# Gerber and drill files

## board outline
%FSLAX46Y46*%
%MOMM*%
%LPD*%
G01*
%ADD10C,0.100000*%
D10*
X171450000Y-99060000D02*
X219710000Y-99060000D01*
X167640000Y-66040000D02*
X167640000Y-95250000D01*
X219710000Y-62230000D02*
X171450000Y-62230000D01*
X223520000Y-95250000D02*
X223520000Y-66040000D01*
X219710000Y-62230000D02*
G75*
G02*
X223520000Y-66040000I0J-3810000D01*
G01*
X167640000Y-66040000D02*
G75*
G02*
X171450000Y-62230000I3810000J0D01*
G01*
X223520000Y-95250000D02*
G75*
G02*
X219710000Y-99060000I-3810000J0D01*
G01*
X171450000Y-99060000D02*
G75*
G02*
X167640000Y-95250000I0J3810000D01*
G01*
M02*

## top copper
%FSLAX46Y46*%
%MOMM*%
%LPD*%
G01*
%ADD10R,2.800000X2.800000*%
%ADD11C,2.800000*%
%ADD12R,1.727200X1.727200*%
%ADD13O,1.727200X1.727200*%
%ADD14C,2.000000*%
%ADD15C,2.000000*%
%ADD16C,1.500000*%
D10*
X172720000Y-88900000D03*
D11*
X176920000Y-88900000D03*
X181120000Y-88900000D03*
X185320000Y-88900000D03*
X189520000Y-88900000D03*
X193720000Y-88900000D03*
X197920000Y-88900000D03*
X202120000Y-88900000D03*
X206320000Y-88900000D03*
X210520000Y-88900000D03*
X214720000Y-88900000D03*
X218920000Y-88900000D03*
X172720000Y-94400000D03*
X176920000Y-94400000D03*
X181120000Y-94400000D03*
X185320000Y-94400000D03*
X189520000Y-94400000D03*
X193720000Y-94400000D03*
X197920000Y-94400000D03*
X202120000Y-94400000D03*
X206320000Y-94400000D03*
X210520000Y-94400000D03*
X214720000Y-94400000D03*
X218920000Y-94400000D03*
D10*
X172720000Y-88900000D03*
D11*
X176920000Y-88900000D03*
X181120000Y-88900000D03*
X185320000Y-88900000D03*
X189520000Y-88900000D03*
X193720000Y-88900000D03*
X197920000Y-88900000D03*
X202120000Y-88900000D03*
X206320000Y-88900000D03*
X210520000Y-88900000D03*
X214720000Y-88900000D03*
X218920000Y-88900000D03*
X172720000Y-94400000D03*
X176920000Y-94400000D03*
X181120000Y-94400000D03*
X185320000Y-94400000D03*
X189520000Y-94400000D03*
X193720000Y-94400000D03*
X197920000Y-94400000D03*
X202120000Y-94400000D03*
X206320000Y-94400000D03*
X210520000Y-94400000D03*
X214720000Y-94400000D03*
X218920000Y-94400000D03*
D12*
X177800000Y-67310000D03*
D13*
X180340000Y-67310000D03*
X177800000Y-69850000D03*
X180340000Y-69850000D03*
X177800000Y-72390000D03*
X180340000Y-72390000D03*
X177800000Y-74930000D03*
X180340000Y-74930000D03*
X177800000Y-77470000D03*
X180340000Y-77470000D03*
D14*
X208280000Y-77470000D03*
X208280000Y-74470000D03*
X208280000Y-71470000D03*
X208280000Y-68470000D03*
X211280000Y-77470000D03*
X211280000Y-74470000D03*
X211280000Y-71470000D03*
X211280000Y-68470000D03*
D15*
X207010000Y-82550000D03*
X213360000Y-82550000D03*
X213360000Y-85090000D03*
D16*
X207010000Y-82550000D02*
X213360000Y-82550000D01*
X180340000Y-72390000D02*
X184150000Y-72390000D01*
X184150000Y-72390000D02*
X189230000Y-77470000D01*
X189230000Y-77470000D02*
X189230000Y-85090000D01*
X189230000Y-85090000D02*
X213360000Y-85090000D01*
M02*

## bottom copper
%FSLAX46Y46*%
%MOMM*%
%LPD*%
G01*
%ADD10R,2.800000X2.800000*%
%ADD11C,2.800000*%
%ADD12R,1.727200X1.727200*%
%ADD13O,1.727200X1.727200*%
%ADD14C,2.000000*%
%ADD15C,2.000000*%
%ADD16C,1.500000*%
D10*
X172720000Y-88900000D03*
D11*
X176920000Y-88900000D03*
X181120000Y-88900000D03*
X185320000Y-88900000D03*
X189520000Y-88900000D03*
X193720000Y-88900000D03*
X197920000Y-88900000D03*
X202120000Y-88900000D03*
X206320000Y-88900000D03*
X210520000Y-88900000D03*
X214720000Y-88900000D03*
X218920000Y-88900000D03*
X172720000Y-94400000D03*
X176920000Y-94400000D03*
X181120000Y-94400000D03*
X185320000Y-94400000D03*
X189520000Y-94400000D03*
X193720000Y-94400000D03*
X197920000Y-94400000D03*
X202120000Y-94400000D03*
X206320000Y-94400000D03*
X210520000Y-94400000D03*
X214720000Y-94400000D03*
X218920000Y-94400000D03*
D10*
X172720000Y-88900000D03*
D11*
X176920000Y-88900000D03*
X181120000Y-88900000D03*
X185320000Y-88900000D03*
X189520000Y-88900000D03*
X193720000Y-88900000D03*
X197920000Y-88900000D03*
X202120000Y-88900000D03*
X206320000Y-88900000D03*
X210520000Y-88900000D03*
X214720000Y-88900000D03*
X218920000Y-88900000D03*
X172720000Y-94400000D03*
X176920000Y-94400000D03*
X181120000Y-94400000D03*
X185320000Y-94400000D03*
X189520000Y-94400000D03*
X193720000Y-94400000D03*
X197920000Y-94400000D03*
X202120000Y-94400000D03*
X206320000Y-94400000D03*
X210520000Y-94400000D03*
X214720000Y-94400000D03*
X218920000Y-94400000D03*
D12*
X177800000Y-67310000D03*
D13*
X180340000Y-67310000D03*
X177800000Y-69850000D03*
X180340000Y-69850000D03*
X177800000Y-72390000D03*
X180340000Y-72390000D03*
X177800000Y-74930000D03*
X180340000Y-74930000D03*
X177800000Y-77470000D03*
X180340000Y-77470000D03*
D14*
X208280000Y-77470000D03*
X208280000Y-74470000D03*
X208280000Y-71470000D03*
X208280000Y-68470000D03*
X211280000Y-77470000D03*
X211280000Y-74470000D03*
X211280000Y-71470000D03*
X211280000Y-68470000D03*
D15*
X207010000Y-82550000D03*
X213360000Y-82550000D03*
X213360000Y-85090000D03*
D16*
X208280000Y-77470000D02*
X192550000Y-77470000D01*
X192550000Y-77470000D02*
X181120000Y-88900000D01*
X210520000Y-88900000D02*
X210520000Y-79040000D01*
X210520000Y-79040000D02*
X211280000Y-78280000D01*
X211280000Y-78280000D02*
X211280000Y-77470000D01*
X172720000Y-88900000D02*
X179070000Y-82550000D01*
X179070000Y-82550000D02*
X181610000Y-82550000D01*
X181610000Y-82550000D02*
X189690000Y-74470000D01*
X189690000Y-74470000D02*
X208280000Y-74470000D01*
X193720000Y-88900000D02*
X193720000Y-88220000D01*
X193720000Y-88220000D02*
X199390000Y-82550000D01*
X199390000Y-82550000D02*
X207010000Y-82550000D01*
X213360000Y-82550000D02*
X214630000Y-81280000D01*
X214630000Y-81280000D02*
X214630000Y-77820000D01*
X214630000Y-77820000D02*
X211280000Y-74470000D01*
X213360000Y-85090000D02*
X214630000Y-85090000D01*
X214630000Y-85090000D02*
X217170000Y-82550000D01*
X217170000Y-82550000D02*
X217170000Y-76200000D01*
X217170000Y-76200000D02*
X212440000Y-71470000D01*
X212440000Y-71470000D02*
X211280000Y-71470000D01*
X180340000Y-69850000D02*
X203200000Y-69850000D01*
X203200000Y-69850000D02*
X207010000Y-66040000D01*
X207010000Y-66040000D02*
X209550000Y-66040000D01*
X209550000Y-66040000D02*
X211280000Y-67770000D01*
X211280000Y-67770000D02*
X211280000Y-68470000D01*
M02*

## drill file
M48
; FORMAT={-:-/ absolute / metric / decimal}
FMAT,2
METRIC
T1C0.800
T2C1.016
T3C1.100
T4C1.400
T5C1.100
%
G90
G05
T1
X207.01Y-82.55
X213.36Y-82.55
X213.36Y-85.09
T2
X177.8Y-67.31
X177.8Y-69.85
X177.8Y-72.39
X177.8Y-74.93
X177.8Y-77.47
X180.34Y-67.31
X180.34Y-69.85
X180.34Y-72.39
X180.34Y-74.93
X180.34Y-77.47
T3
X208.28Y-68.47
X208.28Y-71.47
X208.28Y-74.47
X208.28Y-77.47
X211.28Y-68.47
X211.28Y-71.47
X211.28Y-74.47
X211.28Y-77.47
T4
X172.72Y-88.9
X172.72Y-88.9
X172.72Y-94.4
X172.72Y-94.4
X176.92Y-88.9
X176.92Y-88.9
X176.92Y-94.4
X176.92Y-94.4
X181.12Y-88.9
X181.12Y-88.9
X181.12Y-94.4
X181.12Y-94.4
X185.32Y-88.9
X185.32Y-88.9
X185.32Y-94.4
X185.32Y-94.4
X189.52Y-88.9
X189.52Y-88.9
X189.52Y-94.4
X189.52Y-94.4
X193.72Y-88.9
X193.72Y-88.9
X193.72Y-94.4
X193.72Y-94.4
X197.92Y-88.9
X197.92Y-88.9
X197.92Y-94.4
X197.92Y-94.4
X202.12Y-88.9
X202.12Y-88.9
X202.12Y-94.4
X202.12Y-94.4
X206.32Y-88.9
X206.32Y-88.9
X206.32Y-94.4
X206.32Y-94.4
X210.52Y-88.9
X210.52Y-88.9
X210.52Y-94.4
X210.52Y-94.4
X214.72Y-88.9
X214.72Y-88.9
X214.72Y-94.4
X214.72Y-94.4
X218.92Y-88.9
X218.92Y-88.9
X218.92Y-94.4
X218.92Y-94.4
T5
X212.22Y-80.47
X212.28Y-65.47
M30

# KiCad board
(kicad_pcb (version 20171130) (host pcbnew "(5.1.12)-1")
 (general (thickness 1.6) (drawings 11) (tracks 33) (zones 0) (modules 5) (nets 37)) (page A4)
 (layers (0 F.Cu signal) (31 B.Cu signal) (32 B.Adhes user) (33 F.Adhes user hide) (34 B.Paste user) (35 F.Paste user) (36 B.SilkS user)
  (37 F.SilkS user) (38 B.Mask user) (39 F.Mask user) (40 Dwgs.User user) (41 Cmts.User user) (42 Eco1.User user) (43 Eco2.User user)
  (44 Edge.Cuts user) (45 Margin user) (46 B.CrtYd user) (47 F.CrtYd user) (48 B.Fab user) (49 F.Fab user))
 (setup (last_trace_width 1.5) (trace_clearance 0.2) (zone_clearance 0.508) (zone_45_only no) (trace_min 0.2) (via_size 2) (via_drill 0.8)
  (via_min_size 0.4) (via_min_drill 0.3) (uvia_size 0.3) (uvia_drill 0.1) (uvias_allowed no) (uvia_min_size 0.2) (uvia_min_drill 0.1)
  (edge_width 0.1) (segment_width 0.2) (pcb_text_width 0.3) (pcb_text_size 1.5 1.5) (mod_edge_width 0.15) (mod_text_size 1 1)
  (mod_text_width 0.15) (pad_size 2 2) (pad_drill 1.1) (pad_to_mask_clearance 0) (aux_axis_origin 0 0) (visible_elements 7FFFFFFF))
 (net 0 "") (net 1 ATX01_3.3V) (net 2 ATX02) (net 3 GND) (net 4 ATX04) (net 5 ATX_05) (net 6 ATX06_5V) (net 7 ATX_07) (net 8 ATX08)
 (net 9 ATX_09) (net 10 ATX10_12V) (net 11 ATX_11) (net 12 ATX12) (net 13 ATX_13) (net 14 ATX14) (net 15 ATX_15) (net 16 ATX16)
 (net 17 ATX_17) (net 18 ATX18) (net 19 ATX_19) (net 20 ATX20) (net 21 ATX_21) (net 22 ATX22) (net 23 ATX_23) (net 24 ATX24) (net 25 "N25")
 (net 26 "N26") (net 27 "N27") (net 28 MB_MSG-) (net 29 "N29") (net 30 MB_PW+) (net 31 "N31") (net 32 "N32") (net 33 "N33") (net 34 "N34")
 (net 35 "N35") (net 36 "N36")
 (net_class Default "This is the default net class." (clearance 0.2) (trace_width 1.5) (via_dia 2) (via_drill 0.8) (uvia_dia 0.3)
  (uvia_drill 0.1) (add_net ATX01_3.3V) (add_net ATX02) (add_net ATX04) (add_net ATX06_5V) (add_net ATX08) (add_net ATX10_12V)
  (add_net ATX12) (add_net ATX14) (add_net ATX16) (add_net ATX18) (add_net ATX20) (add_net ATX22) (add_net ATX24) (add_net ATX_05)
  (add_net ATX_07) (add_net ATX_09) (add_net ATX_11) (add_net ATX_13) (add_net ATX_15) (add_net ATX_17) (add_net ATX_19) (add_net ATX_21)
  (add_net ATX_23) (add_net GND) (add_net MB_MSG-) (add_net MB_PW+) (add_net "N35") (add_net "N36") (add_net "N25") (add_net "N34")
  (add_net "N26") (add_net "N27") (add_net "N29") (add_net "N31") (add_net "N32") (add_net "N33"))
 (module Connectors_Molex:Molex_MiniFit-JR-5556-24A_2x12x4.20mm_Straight (layer F.Cu) (at 172.72 88.9)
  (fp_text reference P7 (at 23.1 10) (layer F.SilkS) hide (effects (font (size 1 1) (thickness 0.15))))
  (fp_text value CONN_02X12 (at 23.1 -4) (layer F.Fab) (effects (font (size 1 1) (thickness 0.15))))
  (pad 1 thru_hole rect (at 0 0) (size 2.8 2.8) (drill 1.4) (layers *.Cu *.Mask) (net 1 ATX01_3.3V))
  (pad 2 thru_hole circle (at 4.2 0) (size 2.8 2.8) (drill 1.4) (layers *.Cu *.Mask) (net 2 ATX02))
  (pad 3 thru_hole circle (at 8.4 0) (size 2.8 2.8) (drill 1.4) (layers *.Cu *.Mask) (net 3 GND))
  (pad 4 thru_hole circle (at 12.6 0) (size 2.8 2.8) (drill 1.4) (layers *.Cu *.Mask) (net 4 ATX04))
  (pad 5 thru_hole circle (at 16.8 0) (size 2.8 2.8) (drill 1.4) (layers *.Cu *.Mask) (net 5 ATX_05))
  (pad 6 thru_hole circle (at 21 0) (size 2.8 2.8) (drill 1.4) (layers *.Cu *.Mask) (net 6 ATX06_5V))
  (pad 7 thru_hole circle (at 25.2 0) (size 2.8 2.8) (drill 1.4) (layers *.Cu *.Mask) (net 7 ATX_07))
  (pad 8 thru_hole circle (at 29.4 0) (size 2.8 2.8) (drill 1.4) (layers *.Cu *.Mask) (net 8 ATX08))
  (pad 9 thru_hole circle (at 33.6 0) (size 2.8 2.8) (drill 1.4) (layers *.Cu *.Mask) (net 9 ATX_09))
  (pad 10 thru_hole circle (at 37.8 0) (size 2.8 2.8) (drill 1.4) (layers *.Cu *.Mask) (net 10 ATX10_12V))
  (pad 11 thru_hole circle (at 42 0) (size 2.8 2.8) (drill 1.4) (layers *.Cu *.Mask) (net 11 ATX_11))
  (pad 12 thru_hole circle (at 46.2 0) (size 2.8 2.8) (drill 1.4) (layers *.Cu *.Mask) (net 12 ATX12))
  (pad 13 thru_hole circle (at 0 5.5) (size 2.8 2.8) (drill 1.4) (layers *.Cu *.Mask) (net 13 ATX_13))
  (pad 14 thru_hole circle (at 4.2 5.5) (size 2.8 2.8) (drill 1.4) (layers *.Cu *.Mask) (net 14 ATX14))
  (pad 15 thru_hole circle (at 8.4 5.5) (size 2.8 2.8) (drill 1.4) (layers *.Cu *.Mask) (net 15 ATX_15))
  (pad 16 thru_hole circle (at 12.6 5.5) (size 2.8 2.8) (drill 1.4) (layers *.Cu *.Mask) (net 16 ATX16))
  (pad 17 thru_hole circle (at 16.8 5.5) (size 2.8 2.8) (drill 1.4) (layers *.Cu *.Mask) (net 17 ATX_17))
  (pad 18 thru_hole circle (at 21 5.5) (size 2.8 2.8) (drill 1.4) (layers *.Cu *.Mask) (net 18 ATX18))
  (pad 19 thru_hole circle (at 25.2 5.5) (size 2.8 2.8) (drill 1.4) (layers *.Cu *.Mask) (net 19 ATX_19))
  (pad 20 thru_hole circle (at 29.4 5.5) (size 2.8 2.8) (drill 1.4) (layers *.Cu *.Mask) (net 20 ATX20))
  (pad 21 thru_hole circle (at 33.6 5.5) (size 2.8 2.8) (drill 1.4) (layers *.Cu *.Mask) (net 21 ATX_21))
  (pad 22 thru_hole circle (at 37.8 5.5) (size 2.8 2.8) (drill 1.4) (layers *.Cu *.Mask) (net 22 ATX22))
  (pad 23 thru_hole circle (at 42 5.5) (size 2.8 2.8) (drill 1.4) (layers *.Cu *.Mask) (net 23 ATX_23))
  (pad 24 thru_hole circle (at 46.2 5.5) (size 2.8 2.8) (drill 1.4) (layers *.Cu *.Mask) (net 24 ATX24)))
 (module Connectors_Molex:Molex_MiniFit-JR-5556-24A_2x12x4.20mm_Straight (layer F.Cu) (at 172.72 88.9)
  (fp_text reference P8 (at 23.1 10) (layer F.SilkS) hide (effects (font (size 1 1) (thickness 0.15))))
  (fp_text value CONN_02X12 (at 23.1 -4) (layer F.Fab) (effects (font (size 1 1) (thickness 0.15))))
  (pad 1 thru_hole rect (at 0 0) (size 2.8 2.8) (drill 1.4) (layers *.Cu *.Mask) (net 1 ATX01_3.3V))
  (pad 2 thru_hole circle (at 4.2 0) (size 2.8 2.8) (drill 1.4) (layers *.Cu *.Mask) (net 2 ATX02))
  (pad 3 thru_hole circle (at 8.4 0) (size 2.8 2.8) (drill 1.4) (layers *.Cu *.Mask) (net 3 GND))
  (pad 4 thru_hole circle (at 12.6 0) (size 2.8 2.8) (drill 1.4) (layers *.Cu *.Mask) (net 4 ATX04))
  (pad 5 thru_hole circle (at 16.8 0) (size 2.8 2.8) (drill 1.4) (layers *.Cu *.Mask) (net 5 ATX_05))
  (pad 6 thru_hole circle (at 21 0) (size 2.8 2.8) (drill 1.4) (layers *.Cu *.Mask) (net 6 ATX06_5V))
  (pad 7 thru_hole circle (at 25.2 0) (size 2.8 2.8) (drill 1.4) (layers *.Cu *.Mask) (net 7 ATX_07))
  (pad 8 thru_hole circle (at 29.4 0) (size 2.8 2.8) (drill 1.4) (layers *.Cu *.Mask) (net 8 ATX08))
  (pad 9 thru_hole circle (at 33.6 0) (size 2.8 2.8) (drill 1.4) (layers *.Cu *.Mask) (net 9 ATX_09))
  (pad 10 thru_hole circle (at 37.8 0) (size 2.8 2.8) (drill 1.4) (layers *.Cu *.Mask) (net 10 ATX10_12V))
  (pad 11 thru_hole circle (at 42 0) (size 2.8 2.8) (drill 1.4) (layers *.Cu *.Mask) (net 11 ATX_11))
  (pad 12 thru_hole circle (at 46.2 0) (size 2.8 2.8) (drill 1.4) (layers *.Cu *.Mask) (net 12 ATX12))
  (pad 13 thru_hole circle (at 0 5.5) (size 2.8 2.8) (drill 1.4) (layers *.Cu *.Mask) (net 13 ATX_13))
  (pad 14 thru_hole circle (at 4.2 5.5) (size 2.8 2.8) (drill 1.4) (layers *.Cu *.Mask) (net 14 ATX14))
  (pad 15 thru_hole circle (at 8.4 5.5) (size 2.8 2.8) (drill 1.4) (layers *.Cu *.Mask) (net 15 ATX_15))
  (pad 16 thru_hole circle (at 12.6 5.5) (size 2.8 2.8) (drill 1.4) (layers *.Cu *.Mask) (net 16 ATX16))
  (pad 17 thru_hole circle (at 16.8 5.5) (size 2.8 2.8) (drill 1.4) (layers *.Cu *.Mask) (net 17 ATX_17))
  (pad 18 thru_hole circle (at 21 5.5) (size 2.8 2.8) (drill 1.4) (layers *.Cu *.Mask) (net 18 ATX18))
  (pad 19 thru_hole circle (at 25.2 5.5) (size 2.8 2.8) (drill 1.4) (layers *.Cu *.Mask) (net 19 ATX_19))
  (pad 20 thru_hole circle (at 29.4 5.5) (size 2.8 2.8) (drill 1.4) (layers *.Cu *.Mask) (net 20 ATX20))
  (pad 21 thru_hole circle (at 33.6 5.5) (size 2.8 2.8) (drill 1.4) (layers *.Cu *.Mask) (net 21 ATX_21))
  (pad 22 thru_hole circle (at 37.8 5.5) (size 2.8 2.8) (drill 1.4) (layers *.Cu *.Mask) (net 22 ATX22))
  (pad 23 thru_hole circle (at 42 5.5) (size 2.8 2.8) (drill 1.4) (layers *.Cu *.Mask) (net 23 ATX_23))
  (pad 24 thru_hole circle (at 46.2 5.5) (size 2.8 2.8) (drill 1.4) (layers *.Cu *.Mask) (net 24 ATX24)))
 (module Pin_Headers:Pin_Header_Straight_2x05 (layer F.Cu) (at 177.8 67.31)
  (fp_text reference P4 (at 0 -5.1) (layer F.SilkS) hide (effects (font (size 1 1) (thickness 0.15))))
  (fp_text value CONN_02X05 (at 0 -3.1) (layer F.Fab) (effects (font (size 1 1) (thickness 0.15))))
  (pad 1 thru_hole rect (at 0 0) (size 1.7272 1.7272) (drill 1.016) (layers *.Cu *.Mask F.SilkS) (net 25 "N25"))
  (pad 2 thru_hole oval (at 2.54 0) (size 1.7272 1.7272) (drill 1.016) (layers *.Cu *.Mask F.SilkS) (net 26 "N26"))
  (pad 3 thru_hole oval (at 0 2.54) (size 1.7272 1.7272) (drill 1.016) (layers *.Cu *.Mask F.SilkS) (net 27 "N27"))
  (pad 4 thru_hole oval (at 2.54 2.54) (size 1.7272 1.7272) (drill 1.016) (layers *.Cu *.Mask F.SilkS) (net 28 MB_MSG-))
  (pad 5 thru_hole oval (at 0 5.08) (size 1.7272 1.7272) (drill 1.016) (layers *.Cu *.Mask F.SilkS) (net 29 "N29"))
  (pad 6 thru_hole oval (at 2.54 5.08) (size 1.7272 1.7272) (drill 1.016) (layers *.Cu *.Mask F.SilkS) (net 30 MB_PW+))
  (pad 7 thru_hole oval (at 0 7.62) (size 1.7272 1.7272) (drill 1.016) (layers *.Cu *.Mask F.SilkS) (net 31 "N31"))
  (pad 8 thru_hole oval (at 2.54 7.62) (size 1.7272 1.7272) (drill 1.016) (layers *.Cu *.Mask F.SilkS) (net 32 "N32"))
  (pad 9 thru_hole oval (at 0 10.16) (size 1.7272 1.7272) (drill 1.016) (layers *.Cu *.Mask F.SilkS) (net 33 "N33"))
  (pad 10 thru_hole oval (at 2.54 10.16) (size 1.7272 1.7272) (drill 1.016) (layers *.Cu *.Mask F.SilkS) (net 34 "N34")))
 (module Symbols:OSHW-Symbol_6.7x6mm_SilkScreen (layer F.Cu) (at 193.548 76.2)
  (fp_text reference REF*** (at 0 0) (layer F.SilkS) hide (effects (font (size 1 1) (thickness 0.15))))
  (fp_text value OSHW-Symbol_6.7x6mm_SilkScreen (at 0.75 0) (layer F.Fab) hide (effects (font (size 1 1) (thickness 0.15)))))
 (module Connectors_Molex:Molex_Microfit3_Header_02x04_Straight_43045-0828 (layer F.Cu) (at 208.28 77.47 270)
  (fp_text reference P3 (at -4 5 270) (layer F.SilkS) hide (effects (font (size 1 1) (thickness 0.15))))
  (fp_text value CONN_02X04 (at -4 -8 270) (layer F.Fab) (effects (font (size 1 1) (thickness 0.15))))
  (pad "" np_thru_hole circle (at -12 -4 270) (size 1.1 1.1) (drill 1.1) (layers *.Cu *.Mask F.SilkS))
  (pad 1 thru_hole circle (at 0 0 270) (size 2 2) (drill 1.1) (layers *.Cu *.Mask F.SilkS) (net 3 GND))
  (pad 2 thru_hole circle (at -3 0 270) (size 2 2) (drill 1.1) (layers *.Cu *.Mask F.SilkS) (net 1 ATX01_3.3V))
  (pad 3 thru_hole circle (at -6 0 270) (size 2 2) (drill 1.1) (layers *.Cu *.Mask F.SilkS) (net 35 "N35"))
  (pad 4 thru_hole circle (at -9 0 270) (size 2 2) (drill 1.1) (layers *.Cu *.Mask F.SilkS) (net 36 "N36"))
  (pad 5 thru_hole circle (at 0 -3 270) (size 2 2) (drill 1.1) (layers *.Cu *.Mask F.SilkS) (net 10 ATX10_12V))
  (pad 6 thru_hole circle (at -3 -3 270) (size 2 2) (drill 1.1) (layers *.Cu *.Mask F.SilkS) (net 6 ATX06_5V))
  (pad 7 thru_hole circle (at -6 -3 270) (size 2 2) (drill 1.1) (layers *.Cu *.Mask F.SilkS) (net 30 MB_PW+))
  (pad 8 thru_hole circle (at -9 -3 270) (size 2 2) (drill 1.1) (layers *.Cu *.Mask F.SilkS) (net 28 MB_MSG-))
  (pad "" np_thru_hole circle (at 3 -3.94 270) (size 1.1 1.1) (drill 1.1) (layers *.Cu *.Mask F.SilkS)))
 (gr_line (start 171.45 99.06) (end 219.71 99.06) (angle 90) (layer Edge.Cuts) (width 0.1))
 (gr_line (start 167.64 66.04) (end 167.64 95.25) (angle 90) (layer Edge.Cuts) (width 0.1))
 (gr_line (start 219.71 62.23) (end 171.45 62.23) (angle 90) (layer Edge.Cuts) (width 0.1))
 (gr_line (start 223.52 95.25) (end 223.52 66.04) (angle 90) (layer Edge.Cuts) (width 0.1))
 (gr_arc (start 219.71 66.04) (end 219.71 62.23) (angle 90) (layer Edge.Cuts) (width 0.1))
 (gr_arc (start 171.45 66.04) (end 167.64 66.04) (angle 90) (layer Edge.Cuts) (width 0.1))
 (gr_arc (start 219.71 95.25) (end 223.52 95.25) (angle 90) (layer Edge.Cuts) (width 0.1))
 (gr_arc (start 171.45 95.25) (end 171.45 99.06) (angle 90) (layer Edge.Cuts) (width 0.1))
 (segment (start 208.28 77.47) (end 192.55 77.47) (width 1.5) (layer B.Cu) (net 3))
 (segment (start 192.55 77.47) (end 181.12 88.9) (width 1.5) (layer B.Cu) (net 3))
 (segment (start 210.52 88.9) (end 210.52 79.04) (width 1.5) (layer B.Cu) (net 10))
 (segment (start 210.52 79.04) (end 211.28 78.28) (width 1.5) (layer B.Cu) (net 10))
 (segment (start 211.28 78.28) (end 211.28 77.47) (width 1.5) (layer B.Cu) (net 10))
 (segment (start 172.72 88.9) (end 179.07 82.55) (width 1.5) (layer B.Cu) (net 1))
 (segment (start 179.07 82.55) (end 181.61 82.55) (width 1.5) (layer B.Cu) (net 1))
 (segment (start 181.61 82.55) (end 189.69 74.47) (width 1.5) (layer B.Cu) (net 1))
 (segment (start 189.69 74.47) (end 208.28 74.47) (width 1.5) (layer B.Cu) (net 1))
 (segment (start 193.72 88.9) (end 193.72 88.22) (width 1.5) (layer B.Cu) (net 6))
 (segment (start 193.72 88.22) (end 199.39 82.55) (width 1.5) (layer B.Cu) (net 6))
 (segment (start 199.39 82.55) (end 207.01 82.55) (width 1.5) (layer B.Cu) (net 6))
 (segment (start 207.01 82.55) (end 213.36 82.55) (width 1.5) (layer F.Cu) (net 6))
 (segment (start 213.36 82.55) (end 214.63 81.28) (width 1.5) (layer B.Cu) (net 6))
 (segment (start 214.63 81.28) (end 214.63 77.82) (width 1.5) (layer B.Cu) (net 6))
 (segment (start 214.63 77.82) (end 211.28 74.47) (width 1.5) (layer B.Cu) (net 6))
 (via (at 207.01 82.55) (size 2) (layers F.Cu B.Cu) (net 6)) (via (at 213.36 82.55) (size 2) (layers F.Cu B.Cu) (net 6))
 (segment (start 180.34 72.39) (end 184.15 72.39) (width 1.5) (layer F.Cu) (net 30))
 (segment (start 184.15 72.39) (end 189.23 77.47) (width 1.5) (layer F.Cu) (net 30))
 (segment (start 189.23 77.47) (end 189.23 85.09) (width 1.5) (layer F.Cu) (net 30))
 (segment (start 189.23 85.09) (end 213.36 85.09) (width 1.5) (layer F.Cu) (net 30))
 (segment (start 213.36 85.09) (end 214.63 85.09) (width 1.5) (layer B.Cu) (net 30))
 (segment (start 214.63 85.09) (end 217.17 82.55) (width 1.5) (layer B.Cu) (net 30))
 (segment (start 217.17 82.55) (end 217.17 76.2) (width 1.5) (layer B.Cu) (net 30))
 (segment (start 217.17 76.2) (end 212.44 71.47) (width 1.5) (layer B.Cu) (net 30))
 (segment (start 212.44 71.47) (end 211.28 71.47) (width 1.5) (layer B.Cu) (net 30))
 (via (at 213.36 85.09) (size 2) (layers F.Cu B.Cu) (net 30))
 (segment (start 180.34 69.85) (end 203.2 69.85) (width 1.5) (layer B.Cu) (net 28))
 (segment (start 203.2 69.85) (end 207.01 66.04) (width 1.5) (layer B.Cu) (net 28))
 (segment (start 207.01 66.04) (end 209.55 66.04) (width 1.5) (layer B.Cu) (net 28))
 (segment (start 209.55 66.04) (end 211.28 67.77) (width 1.5) (layer B.Cu) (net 28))
 (segment (start 211.28 67.77) (end 211.28 68.47) (width 1.5) (layer B.Cu) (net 28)))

